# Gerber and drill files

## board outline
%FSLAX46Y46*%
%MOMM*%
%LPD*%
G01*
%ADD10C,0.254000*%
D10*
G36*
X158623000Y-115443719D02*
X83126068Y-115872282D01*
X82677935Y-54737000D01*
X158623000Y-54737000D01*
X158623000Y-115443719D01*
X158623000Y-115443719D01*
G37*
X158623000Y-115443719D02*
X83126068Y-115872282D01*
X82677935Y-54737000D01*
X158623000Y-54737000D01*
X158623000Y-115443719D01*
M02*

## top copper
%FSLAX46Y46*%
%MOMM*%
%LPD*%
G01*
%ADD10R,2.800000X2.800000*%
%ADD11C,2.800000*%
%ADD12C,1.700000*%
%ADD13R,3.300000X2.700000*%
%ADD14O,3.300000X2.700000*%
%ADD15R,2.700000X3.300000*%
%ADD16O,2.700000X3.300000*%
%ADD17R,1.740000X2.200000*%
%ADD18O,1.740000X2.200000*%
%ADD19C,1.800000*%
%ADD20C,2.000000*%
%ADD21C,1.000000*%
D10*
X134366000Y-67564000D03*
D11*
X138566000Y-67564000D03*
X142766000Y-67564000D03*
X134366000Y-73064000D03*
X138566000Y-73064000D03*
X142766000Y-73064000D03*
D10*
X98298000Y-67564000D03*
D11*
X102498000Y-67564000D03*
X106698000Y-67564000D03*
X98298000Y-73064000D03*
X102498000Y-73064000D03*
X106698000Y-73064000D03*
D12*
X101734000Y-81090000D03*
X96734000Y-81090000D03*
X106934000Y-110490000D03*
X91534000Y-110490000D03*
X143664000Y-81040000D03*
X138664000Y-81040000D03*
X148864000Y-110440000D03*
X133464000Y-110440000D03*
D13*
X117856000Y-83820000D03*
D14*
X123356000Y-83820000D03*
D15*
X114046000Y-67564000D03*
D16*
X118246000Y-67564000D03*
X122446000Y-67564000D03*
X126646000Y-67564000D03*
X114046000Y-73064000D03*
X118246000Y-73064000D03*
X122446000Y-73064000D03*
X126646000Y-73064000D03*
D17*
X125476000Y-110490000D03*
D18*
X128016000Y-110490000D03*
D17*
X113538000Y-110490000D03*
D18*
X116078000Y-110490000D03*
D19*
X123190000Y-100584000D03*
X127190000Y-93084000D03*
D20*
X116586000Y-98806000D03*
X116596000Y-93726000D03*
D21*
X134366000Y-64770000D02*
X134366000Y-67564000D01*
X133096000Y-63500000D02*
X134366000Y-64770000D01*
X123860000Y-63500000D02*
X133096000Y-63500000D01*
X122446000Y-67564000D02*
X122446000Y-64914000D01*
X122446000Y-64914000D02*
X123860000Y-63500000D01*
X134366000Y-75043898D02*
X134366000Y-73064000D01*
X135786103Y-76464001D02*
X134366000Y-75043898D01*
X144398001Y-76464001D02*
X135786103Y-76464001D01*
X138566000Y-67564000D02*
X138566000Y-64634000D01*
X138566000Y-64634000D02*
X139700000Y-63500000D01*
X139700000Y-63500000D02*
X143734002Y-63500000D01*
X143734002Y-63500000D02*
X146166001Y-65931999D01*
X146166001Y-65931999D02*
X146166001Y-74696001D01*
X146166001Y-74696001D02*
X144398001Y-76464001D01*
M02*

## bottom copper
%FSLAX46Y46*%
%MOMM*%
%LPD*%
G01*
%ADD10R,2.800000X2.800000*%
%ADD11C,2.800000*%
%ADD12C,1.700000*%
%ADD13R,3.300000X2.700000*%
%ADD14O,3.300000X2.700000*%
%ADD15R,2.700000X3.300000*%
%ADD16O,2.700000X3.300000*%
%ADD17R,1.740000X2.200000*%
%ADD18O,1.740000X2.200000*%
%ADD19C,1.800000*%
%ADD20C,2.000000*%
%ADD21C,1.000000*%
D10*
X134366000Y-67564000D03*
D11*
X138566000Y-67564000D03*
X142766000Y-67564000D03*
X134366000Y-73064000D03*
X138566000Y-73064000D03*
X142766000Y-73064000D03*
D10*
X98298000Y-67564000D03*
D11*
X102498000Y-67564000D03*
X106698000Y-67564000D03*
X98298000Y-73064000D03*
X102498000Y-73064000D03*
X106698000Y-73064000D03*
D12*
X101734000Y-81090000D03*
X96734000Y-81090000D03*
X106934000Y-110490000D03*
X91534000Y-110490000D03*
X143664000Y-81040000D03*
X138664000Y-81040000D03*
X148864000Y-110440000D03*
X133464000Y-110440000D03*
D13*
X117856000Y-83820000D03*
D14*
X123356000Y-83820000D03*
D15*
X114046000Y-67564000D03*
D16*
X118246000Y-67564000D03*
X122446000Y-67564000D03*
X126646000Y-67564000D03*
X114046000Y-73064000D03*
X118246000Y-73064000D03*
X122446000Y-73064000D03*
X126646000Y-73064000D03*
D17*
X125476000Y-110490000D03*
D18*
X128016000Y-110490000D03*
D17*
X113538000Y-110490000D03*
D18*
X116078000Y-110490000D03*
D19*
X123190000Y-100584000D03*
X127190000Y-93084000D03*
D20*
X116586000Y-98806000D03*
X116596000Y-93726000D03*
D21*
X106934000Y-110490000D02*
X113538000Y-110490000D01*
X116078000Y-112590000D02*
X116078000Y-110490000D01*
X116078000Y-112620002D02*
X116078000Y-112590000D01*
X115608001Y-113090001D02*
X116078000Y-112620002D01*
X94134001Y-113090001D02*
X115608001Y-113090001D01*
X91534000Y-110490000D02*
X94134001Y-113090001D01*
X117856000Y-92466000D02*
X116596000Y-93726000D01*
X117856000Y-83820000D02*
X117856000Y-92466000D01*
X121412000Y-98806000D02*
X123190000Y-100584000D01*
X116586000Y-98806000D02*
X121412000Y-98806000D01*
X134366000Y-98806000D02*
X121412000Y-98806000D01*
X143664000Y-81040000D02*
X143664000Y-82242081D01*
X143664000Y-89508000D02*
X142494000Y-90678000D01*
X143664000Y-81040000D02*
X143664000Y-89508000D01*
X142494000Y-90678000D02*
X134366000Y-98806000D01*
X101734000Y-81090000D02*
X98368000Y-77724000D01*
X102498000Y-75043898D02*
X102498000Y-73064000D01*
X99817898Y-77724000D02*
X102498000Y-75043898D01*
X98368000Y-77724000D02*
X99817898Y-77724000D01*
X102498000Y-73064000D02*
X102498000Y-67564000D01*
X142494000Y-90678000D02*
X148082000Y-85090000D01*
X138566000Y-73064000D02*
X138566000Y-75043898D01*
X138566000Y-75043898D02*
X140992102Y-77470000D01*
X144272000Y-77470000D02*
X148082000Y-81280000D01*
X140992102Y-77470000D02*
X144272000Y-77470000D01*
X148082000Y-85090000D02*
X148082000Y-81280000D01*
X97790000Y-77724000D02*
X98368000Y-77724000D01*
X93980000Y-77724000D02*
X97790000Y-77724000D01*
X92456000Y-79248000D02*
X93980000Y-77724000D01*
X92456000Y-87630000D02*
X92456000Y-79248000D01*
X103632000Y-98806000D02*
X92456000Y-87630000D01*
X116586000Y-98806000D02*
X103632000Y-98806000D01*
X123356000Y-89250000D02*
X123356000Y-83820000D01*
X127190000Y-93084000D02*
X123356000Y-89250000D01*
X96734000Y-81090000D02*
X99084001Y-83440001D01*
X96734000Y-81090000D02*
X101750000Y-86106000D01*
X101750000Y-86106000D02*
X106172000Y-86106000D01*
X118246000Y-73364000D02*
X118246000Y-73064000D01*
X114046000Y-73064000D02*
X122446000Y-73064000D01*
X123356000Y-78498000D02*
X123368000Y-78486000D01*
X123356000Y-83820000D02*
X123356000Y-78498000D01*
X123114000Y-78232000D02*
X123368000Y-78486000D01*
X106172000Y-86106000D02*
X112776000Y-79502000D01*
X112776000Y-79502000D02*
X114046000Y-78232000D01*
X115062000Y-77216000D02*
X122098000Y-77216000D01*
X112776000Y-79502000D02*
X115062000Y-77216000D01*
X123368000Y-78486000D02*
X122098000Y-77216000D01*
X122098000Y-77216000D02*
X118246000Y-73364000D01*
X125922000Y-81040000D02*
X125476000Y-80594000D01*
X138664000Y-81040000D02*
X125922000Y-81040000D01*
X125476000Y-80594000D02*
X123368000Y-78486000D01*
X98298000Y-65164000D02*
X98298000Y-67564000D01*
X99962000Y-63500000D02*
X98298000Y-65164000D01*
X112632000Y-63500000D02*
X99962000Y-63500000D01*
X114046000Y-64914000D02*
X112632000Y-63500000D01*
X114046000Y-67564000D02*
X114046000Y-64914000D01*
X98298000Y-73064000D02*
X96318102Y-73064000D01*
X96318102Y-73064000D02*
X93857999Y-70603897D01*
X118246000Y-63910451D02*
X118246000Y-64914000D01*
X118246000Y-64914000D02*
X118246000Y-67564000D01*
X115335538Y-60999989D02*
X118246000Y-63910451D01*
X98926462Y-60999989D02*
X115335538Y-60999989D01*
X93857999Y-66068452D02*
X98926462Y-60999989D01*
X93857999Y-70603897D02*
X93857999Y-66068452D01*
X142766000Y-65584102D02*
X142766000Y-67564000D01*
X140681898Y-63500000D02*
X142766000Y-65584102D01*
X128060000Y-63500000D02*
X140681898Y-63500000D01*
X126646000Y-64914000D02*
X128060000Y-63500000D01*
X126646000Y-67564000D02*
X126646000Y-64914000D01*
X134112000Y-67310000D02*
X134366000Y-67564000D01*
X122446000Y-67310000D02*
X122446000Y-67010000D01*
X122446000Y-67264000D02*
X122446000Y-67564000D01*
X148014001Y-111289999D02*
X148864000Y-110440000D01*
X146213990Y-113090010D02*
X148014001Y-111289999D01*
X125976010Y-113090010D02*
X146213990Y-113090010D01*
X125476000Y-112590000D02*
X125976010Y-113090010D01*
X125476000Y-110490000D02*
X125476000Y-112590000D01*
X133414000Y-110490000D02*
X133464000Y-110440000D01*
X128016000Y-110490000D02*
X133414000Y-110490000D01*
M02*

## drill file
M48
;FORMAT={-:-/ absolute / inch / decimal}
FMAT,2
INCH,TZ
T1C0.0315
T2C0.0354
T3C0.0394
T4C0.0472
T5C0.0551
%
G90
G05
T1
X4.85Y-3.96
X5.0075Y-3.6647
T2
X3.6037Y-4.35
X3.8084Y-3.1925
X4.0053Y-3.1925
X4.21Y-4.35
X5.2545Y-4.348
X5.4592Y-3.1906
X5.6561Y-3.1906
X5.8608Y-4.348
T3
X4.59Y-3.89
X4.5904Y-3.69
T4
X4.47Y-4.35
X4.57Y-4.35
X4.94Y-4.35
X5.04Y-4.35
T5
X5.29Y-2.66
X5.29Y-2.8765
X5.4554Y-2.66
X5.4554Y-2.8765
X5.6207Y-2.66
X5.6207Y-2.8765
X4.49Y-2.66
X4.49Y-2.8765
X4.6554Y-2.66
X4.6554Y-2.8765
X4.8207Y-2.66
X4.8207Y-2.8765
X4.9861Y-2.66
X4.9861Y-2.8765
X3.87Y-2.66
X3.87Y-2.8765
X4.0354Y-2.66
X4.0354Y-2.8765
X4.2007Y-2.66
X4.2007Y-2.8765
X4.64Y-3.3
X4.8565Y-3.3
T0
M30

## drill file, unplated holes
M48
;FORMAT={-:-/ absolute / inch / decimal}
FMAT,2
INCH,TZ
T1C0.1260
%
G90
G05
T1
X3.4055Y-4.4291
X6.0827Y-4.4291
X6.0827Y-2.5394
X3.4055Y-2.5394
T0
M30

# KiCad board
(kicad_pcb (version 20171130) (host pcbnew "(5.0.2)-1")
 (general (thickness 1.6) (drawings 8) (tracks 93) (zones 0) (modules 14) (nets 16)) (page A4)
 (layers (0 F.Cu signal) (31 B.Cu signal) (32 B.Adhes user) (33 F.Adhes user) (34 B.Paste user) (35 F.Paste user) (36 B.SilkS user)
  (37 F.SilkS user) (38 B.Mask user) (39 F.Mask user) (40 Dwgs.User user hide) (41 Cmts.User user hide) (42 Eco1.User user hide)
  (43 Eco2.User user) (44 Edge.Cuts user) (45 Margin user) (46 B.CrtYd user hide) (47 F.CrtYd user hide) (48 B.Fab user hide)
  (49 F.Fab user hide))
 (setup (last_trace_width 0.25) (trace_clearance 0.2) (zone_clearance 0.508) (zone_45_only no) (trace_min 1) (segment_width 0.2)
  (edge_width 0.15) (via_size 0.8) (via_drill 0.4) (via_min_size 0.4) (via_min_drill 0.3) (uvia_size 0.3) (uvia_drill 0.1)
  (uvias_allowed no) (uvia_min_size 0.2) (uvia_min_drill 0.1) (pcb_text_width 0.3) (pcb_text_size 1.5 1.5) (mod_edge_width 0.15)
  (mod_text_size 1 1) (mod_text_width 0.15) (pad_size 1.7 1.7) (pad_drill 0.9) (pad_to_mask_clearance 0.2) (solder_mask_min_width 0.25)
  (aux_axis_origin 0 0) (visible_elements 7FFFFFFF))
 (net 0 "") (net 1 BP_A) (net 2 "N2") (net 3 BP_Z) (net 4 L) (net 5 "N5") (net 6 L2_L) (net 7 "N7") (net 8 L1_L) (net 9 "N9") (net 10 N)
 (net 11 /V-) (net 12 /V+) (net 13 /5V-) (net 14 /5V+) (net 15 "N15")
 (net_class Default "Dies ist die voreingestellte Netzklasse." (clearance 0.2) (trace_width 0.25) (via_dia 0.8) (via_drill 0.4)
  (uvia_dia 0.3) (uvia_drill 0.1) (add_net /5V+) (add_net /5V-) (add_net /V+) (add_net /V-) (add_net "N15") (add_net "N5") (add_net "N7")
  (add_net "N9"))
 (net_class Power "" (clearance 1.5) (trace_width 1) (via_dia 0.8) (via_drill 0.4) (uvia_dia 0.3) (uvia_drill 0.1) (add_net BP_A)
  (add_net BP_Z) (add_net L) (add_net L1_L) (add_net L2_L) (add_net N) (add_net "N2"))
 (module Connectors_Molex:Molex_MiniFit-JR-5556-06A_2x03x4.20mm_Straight (layer F.Cu) (at 134.366 67.564)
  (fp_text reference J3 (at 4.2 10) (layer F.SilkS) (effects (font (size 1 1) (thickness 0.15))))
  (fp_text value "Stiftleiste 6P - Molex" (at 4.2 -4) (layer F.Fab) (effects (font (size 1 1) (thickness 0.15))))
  (pad 1 thru_hole rect (at 0 0) (size 2.8 2.8) (drill 1.4) (layers *.Cu *.Mask) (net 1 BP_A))
  (pad 2 thru_hole circle (at 4.2 0) (size 2.8 2.8) (drill 1.4) (layers *.Cu *.Mask) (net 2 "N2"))
  (pad 3 thru_hole circle (at 8.4 0) (size 2.8 2.8) (drill 1.4) (layers *.Cu *.Mask) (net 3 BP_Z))
  (pad 4 thru_hole circle (at 0 5.5) (size 2.8 2.8) (drill 1.4) (layers *.Cu *.Mask) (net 2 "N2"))
  (pad 5 thru_hole circle (at 4.2 5.5) (size 2.8 2.8) (drill 1.4) (layers *.Cu *.Mask) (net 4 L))
  (pad 6 thru_hole circle (at 8.4 5.5) (size 2.8 2.8) (drill 1.4) (layers *.Cu *.Mask) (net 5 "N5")))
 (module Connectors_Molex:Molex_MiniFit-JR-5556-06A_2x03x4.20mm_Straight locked (layer F.Cu) (at 98.298 67.564)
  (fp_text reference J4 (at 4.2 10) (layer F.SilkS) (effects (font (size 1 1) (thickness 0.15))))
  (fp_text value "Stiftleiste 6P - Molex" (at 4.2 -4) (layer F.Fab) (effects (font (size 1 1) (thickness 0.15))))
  (pad 1 thru_hole rect (at 0 0) (size 2.8 2.8) (drill 1.4) (layers *.Cu *.Mask) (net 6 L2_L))
  (pad 2 thru_hole circle (at 4.2 0) (size 2.8 2.8) (drill 1.4) (layers *.Cu *.Mask) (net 4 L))
  (pad 3 thru_hole circle (at 8.4 0) (size 2.8 2.8) (drill 1.4) (layers *.Cu *.Mask) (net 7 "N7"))
  (pad 4 thru_hole circle (at 0 5.5) (size 2.8 2.8) (drill 1.4) (layers *.Cu *.Mask) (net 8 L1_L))
  (pad 5 thru_hole circle (at 4.2 5.5) (size 2.8 2.8) (drill 1.4) (layers *.Cu *.Mask) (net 4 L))
  (pad 6 thru_hole circle (at 8.4 5.5) (size 2.8 2.8) (drill 1.4) (layers *.Cu *.Mask) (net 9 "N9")))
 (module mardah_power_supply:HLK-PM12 (layer F.Cu) (at 89.134 78.79 270)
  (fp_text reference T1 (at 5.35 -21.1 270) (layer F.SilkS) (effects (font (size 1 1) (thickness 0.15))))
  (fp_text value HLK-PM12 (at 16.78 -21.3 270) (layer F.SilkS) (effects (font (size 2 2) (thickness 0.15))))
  (pad 1 thru_hole circle (at 2.3 -12.6 270) (size 1.7 1.7) (drill 0.9) (layers *.Cu *.Mask F.SilkS) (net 4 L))
  (pad 2 thru_hole circle (at 2.3 -7.6 270) (size 1.7 1.7) (drill 0.9) (layers *.Cu *.Mask F.SilkS) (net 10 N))
  (pad 3 thru_hole circle (at 31.7 -17.8 270) (size 1.7 1.7) (drill 0.9) (layers *.Cu *.Mask F.SilkS) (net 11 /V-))
  (pad 4 thru_hole circle (at 31.7 -2.4 270) (size 1.7 1.7) (drill 0.9) (layers *.Cu *.Mask F.SilkS) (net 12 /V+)))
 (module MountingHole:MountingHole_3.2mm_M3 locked (layer F.Cu) (at 154.5 64.5)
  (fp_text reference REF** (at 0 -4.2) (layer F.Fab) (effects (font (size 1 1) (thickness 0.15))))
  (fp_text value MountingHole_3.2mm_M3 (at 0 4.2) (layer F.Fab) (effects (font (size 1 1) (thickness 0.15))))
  (pad 1 np_thru_hole circle (at 0 0) (size 3.2 3.2) (drill 3.2) (layers *.Cu *.Mask)))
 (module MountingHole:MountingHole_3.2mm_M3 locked (layer F.Cu) (at 154.5 112.5)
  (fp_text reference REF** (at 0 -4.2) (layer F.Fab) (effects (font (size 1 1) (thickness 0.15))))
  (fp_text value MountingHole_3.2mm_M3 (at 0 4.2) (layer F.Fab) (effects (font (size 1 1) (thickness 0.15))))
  (pad 1 np_thru_hole circle (at 0 0) (size 3.2 3.2) (drill 3.2) (layers *.Cu *.Mask)))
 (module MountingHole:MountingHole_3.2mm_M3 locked (layer F.Cu) (at 86.5 112.5)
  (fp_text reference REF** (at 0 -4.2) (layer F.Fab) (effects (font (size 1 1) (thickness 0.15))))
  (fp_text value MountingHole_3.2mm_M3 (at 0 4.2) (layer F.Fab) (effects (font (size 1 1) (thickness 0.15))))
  (pad 1 np_thru_hole circle (at 0 0) (size 3.2 3.2) (drill 3.2) (layers *.Cu *.Mask)))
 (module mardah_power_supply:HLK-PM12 (layer F.Cu) (at 131.064 78.74 270)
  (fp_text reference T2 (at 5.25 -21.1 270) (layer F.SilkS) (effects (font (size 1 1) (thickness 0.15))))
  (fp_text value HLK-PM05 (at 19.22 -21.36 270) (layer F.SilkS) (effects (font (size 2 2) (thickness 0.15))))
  (pad 1 thru_hole circle (at 2.3 -12.6 270) (size 1.7 1.7) (drill 0.9) (layers *.Cu *.Mask F.SilkS) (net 4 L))
  (pad 2 thru_hole circle (at 2.3 -7.6 270) (size 1.7 1.7) (drill 0.9) (layers *.Cu *.Mask F.SilkS) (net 10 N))
  (pad 3 thru_hole circle (at 31.7 -17.8 270) (size 1.7 1.7) (drill 0.9) (layers *.Cu *.Mask F.SilkS) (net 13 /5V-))
  (pad 4 thru_hole circle (at 31.7 -2.4 270) (size 1.7 1.7) (drill 0.9) (layers *.Cu *.Mask F.SilkS) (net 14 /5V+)))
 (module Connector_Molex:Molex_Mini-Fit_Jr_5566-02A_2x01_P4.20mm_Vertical (layer F.Cu) (at 117.856 83.82 90)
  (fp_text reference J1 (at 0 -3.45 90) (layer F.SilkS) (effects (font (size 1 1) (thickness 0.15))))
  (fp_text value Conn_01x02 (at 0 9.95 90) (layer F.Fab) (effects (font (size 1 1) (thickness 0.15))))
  (pad 1 thru_hole rect (at 0 0 90) (size 2.7 3.3) (drill 1.4) (layers *.Cu *.Mask) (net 4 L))
  (pad 2 thru_hole oval (at 0 5.5 90) (size 2.7 3.3) (drill 1.4) (layers *.Cu *.Mask) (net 10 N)))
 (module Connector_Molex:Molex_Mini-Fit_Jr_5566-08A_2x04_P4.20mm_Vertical (layer F.Cu) (at 114.046 67.564)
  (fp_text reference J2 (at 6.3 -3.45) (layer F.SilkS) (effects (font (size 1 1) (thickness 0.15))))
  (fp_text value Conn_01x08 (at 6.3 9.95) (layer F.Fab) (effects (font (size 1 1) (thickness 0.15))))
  (pad 1 thru_hole rect (at 0 0) (size 2.7 3.3) (drill 1.4) (layers *.Cu *.Mask) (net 6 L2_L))
  (pad 2 thru_hole oval (at 4.2 0) (size 2.7 3.3) (drill 1.4) (layers *.Cu *.Mask) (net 8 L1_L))
  (pad 3 thru_hole oval (at 8.4 0) (size 2.7 3.3) (drill 1.4) (layers *.Cu *.Mask) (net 1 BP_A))
  (pad 4 thru_hole oval (at 12.6 0) (size 2.7 3.3) (drill 1.4) (layers *.Cu *.Mask) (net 3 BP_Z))
  (pad 5 thru_hole oval (at 0 5.5) (size 2.7 3.3) (drill 1.4) (layers *.Cu *.Mask) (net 10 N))
  (pad 6 thru_hole oval (at 4.2 5.5) (size 2.7 3.3) (drill 1.4) (layers *.Cu *.Mask) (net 10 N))
  (pad 7 thru_hole oval (at 8.4 5.5) (size 2.7 3.3) (drill 1.4) (layers *.Cu *.Mask) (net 10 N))
  (pad 8 thru_hole oval (at 12.6 5.5) (size 2.7 3.3) (drill 1.4) (layers *.Cu *.Mask) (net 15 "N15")))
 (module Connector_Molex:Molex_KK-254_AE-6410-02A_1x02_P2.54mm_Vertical (layer F.Cu) (at 125.476 110.49)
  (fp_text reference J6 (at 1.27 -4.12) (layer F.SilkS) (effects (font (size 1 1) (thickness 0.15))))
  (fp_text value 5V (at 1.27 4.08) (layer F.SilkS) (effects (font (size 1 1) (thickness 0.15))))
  (pad 1 thru_hole rect (at 0 0) (size 1.74 2.2) (drill 1.2) (layers *.Cu *.Mask) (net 13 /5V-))
  (pad 2 thru_hole oval (at 2.54 0) (size 1.74 2.2) (drill 1.2) (layers *.Cu *.Mask) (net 14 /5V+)))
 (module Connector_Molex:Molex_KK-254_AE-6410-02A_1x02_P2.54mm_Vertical (layer F.Cu) (at 113.538 110.49)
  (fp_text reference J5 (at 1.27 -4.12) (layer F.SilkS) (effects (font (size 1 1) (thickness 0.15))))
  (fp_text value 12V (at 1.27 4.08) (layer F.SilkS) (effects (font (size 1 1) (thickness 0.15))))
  (pad 1 thru_hole rect (at 0 0) (size 1.74 2.2) (drill 1.2) (layers *.Cu *.Mask) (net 11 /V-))
  (pad 2 thru_hole oval (at 2.54 0) (size 1.74 2.2) (drill 1.2) (layers *.Cu *.Mask) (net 12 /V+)))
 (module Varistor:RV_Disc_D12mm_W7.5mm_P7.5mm (layer F.Cu) (at 123.19 100.584 90)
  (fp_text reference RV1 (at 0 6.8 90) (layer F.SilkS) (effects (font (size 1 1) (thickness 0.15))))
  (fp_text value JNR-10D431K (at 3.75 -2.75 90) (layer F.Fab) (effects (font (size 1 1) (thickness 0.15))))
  (pad 1 thru_hole circle (at 0 0 90) (size 1.8 1.8) (drill 0.8) (layers *.Cu *.Mask) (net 4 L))
  (pad 2 thru_hole circle (at 7.5 4 90) (size 1.8 1.8) (drill 0.8) (layers *.Cu *.Mask) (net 10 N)))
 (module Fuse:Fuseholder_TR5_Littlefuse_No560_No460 (layer F.Cu) (at 116.586 98.806 90)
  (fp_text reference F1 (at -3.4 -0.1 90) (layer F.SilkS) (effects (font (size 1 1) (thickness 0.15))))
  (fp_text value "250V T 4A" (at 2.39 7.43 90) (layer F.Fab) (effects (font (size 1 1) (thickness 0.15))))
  (pad 1 thru_hole circle (at 0 0 90) (size 2 2) (drill 1) (layers *.Cu *.Mask) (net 4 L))
  (pad 2 thru_hole circle (at 5.08 0.01 90) (size 2 2) (drill 1) (layers *.Cu *.Mask) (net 4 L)))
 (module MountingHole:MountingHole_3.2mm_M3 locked (layer F.Cu) (at 86.5 64.5)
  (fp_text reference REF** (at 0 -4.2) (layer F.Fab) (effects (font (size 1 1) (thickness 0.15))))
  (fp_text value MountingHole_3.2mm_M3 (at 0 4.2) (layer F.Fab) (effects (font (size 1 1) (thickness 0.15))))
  (pad 1 np_thru_hole circle (at 0 0) (size 3.2 3.2) (drill 3.2) (layers *.Cu *.Mask)))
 (segment (start 106.934 110.49) (end 113.538 110.49) (width 1) (layer B.Cu) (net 11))
 (segment (start 116.078 112.59) (end 116.078 110.49) (width 1) (layer B.Cu) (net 12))
 (segment (start 116.078 112.620002) (end 116.078 112.59) (width 1) (layer B.Cu) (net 12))
 (segment (start 115.608001 113.090001) (end 116.078 112.620002) (width 1) (layer B.Cu) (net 12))
 (segment (start 94.134001 113.090001) (end 115.608001 113.090001) (width 1) (layer B.Cu) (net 12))
 (segment (start 91.534 110.49) (end 94.134001 113.090001) (width 1) (layer B.Cu) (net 12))
 (segment (start 117.856 92.466) (end 116.596 93.726) (width 1) (layer B.Cu) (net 4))
 (segment (start 117.856 83.82) (end 117.856 92.466) (width 1) (layer B.Cu) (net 4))
 (segment (start 121.412 98.806) (end 123.19 100.584) (width 1) (layer B.Cu) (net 4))
 (segment (start 116.586 98.806) (end 121.412 98.806) (width 1) (layer B.Cu) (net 4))
 (segment (start 134.366 98.806) (end 121.412 98.806) (width 1) (layer B.Cu) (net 4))
 (segment (start 143.664 81.04) (end 143.664 82.242081) (width 1) (layer B.Cu) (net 4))
 (segment (start 143.664 89.508) (end 142.494 90.678) (width 1) (layer B.Cu) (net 4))
 (segment (start 143.664 81.04) (end 143.664 89.508) (width 1) (layer B.Cu) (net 4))
 (segment (start 142.494 90.678) (end 134.366 98.806) (width 1) (layer B.Cu) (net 4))
 (segment (start 101.734 81.09) (end 98.368 77.724) (width 1) (layer B.Cu) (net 4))
 (segment (start 102.498 75.043898) (end 102.498 73.064) (width 1) (layer B.Cu) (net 4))
 (segment (start 99.817898 77.724) (end 102.498 75.043898) (width 1) (layer B.Cu) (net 4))
 (segment (start 98.368 77.724) (end 99.817898 77.724) (width 1) (layer B.Cu) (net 4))
 (segment (start 102.498 73.064) (end 102.498 67.564) (width 1) (layer B.Cu) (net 4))
 (segment (start 142.494 90.678) (end 148.082 85.09) (width 1) (layer B.Cu) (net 4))
 (segment (start 138.566 73.064) (end 138.566 75.043898) (width 1) (layer B.Cu) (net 4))
 (segment (start 138.566 75.043898) (end 140.992102 77.47) (width 1) (layer B.Cu) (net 4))
 (segment (start 144.272 77.47) (end 148.082 81.28) (width 1) (layer B.Cu) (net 4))
 (segment (start 140.992102 77.47) (end 144.272 77.47) (width 1) (layer B.Cu) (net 4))
 (segment (start 148.082 85.09) (end 148.082 81.28) (width 1) (layer B.Cu) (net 4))
 (segment (start 97.79 77.724) (end 98.368 77.724) (width 1) (layer B.Cu) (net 4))
 (segment (start 93.98 77.724) (end 97.79 77.724) (width 1) (layer B.Cu) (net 4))
 (segment (start 92.456 79.248) (end 93.98 77.724) (width 1) (layer B.Cu) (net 4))
 (segment (start 92.456 87.63) (end 92.456 79.248) (width 1) (layer B.Cu) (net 4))
 (segment (start 103.632 98.806) (end 92.456 87.63) (width 1) (layer B.Cu) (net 4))
 (segment (start 116.586 98.806) (end 103.632 98.806) (width 1) (layer B.Cu) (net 4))
 (segment (start 123.356 89.25) (end 123.356 83.82) (width 1) (layer B.Cu) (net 10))
 (segment (start 127.19 93.084) (end 123.356 89.25) (width 1) (layer B.Cu) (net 10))
 (segment (start 96.734 81.09) (end 99.084001 83.440001) (width 1) (layer B.Cu) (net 10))
 (segment (start 96.734 81.09) (end 101.75 86.106) (width 1) (layer B.Cu) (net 10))
 (segment (start 101.75 86.106) (end 106.172 86.106) (width 1) (layer B.Cu) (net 10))
 (segment (start 118.246 73.364) (end 118.246 73.064) (width 1) (layer B.Cu) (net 10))
 (segment (start 114.046 73.064) (end 122.446 73.064) (width 1) (layer B.Cu) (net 10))
 (segment (start 123.356 78.498) (end 123.368 78.486) (width 1) (layer B.Cu) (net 10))
 (segment (start 123.356 83.82) (end 123.356 78.498) (width 1) (layer B.Cu) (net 10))
 (segment (start 123.114 78.232) (end 123.368 78.486) (width 1) (layer B.Cu) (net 10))
 (segment (start 106.172 86.106) (end 112.776 79.502) (width 1) (layer B.Cu) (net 10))
 (segment (start 112.776 79.502) (end 114.046 78.232) (width 1) (layer B.Cu) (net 10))
 (segment (start 115.062 77.216) (end 122.098 77.216) (width 1) (layer B.Cu) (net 10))
 (segment (start 112.776 79.502) (end 115.062 77.216) (width 1) (layer B.Cu) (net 10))
 (segment (start 123.368 78.486) (end 122.098 77.216) (width 1) (layer B.Cu) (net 10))
 (segment (start 122.098 77.216) (end 118.246 73.364) (width 1) (layer B.Cu) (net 10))
 (segment (start 125.922 81.04) (end 125.476 80.594) (width 1) (layer B.Cu) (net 10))
 (segment (start 138.664 81.04) (end 125.922 81.04) (width 1) (layer B.Cu) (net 10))
 (segment (start 125.476 80.594) (end 123.368 78.486) (width 1) (layer B.Cu) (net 10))
 (segment (start 98.298 65.164) (end 98.298 67.564) (width 1) (layer B.Cu) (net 6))
 (segment (start 99.962 63.5) (end 98.298 65.164) (width 1) (layer B.Cu) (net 6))
 (segment (start 112.632 63.5) (end 99.962 63.5) (width 1) (layer B.Cu) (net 6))
 (segment (start 114.046 64.914) (end 112.632 63.5) (width 1) (layer B.Cu) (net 6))
 (segment (start 114.046 67.564) (end 114.046 64.914) (width 1) (layer B.Cu) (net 6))
 (segment (start 98.298 73.064) (end 96.318102 73.064) (width 1) (layer B.Cu) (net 8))
 (segment (start 96.318102 73.064) (end 93.857999 70.603897) (width 1) (layer B.Cu) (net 8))
 (segment (start 118.246 63.910451) (end 118.246 64.914) (width 1) (layer B.Cu) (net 8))
 (segment (start 118.246 64.914) (end 118.246 67.564) (width 1) (layer B.Cu) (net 8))
 (segment (start 115.335538 60.999989) (end 118.246 63.910451) (width 1) (layer B.Cu) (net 8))
 (segment (start 98.926462 60.999989) (end 115.335538 60.999989) (width 1) (layer B.Cu) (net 8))
 (segment (start 93.857999 66.068452) (end 98.926462 60.999989) (width 1) (layer B.Cu) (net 8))
 (segment (start 93.857999 70.603897) (end 93.857999 66.068452) (width 1) (layer B.Cu) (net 8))
 (segment (start 142.766 65.584102) (end 142.766 67.564) (width 1) (layer B.Cu) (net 3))
 (segment (start 140.681898 63.5) (end 142.766 65.584102) (width 1) (layer B.Cu) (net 3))
 (segment (start 128.06 63.5) (end 140.681898 63.5) (width 1) (layer B.Cu) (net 3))
 (segment (start 126.646 64.914) (end 128.06 63.5) (width 1) (layer B.Cu) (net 3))
 (segment (start 126.646 67.564) (end 126.646 64.914) (width 1) (layer B.Cu) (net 3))
 (segment (start 134.112 67.31) (end 134.366 67.564) (width 1) (layer B.Cu) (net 1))
 (segment (start 122.446 67.31) (end 122.446 67.01) (width 1) (layer B.Cu) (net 1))
 (segment (start 122.446 67.264) (end 122.446 67.564) (width 1) (layer B.Cu) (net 1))
 (segment (start 134.366 64.77) (end 134.366 67.564) (width 1) (layer F.Cu) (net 1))
 (segment (start 133.096 63.5) (end 134.366 64.77) (width 1) (layer F.Cu) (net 1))
 (segment (start 123.86 63.5) (end 133.096 63.5) (width 1) (layer F.Cu) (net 1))
 (segment (start 122.446 67.564) (end 122.446 64.914) (width 1) (layer F.Cu) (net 1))
 (segment (start 122.446 64.914) (end 123.86 63.5) (width 1) (layer F.Cu) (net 1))
 (segment (start 148.014001 111.289999) (end 148.864 110.44) (width 1) (layer B.Cu) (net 13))
 (segment (start 146.21399 113.09001) (end 148.014001 111.289999) (width 1) (layer B.Cu) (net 13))
 (segment (start 125.97601 113.09001) (end 146.21399 113.09001) (width 1) (layer B.Cu) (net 13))
 (segment (start 125.476 112.59) (end 125.97601 113.09001) (width 1) (layer B.Cu) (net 13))
 (segment (start 125.476 110.49) (end 125.476 112.59) (width 1) (layer B.Cu) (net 13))
 (segment (start 133.414 110.49) (end 133.464 110.44) (width 1) (layer B.Cu) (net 14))
 (segment (start 128.016 110.49) (end 133.414 110.49) (width 1) (layer B.Cu) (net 14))
 (segment (start 134.366 75.043898) (end 134.366 73.064) (width 1) (layer F.Cu) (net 2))
 (segment (start 135.786103 76.464001) (end 134.366 75.043898) (width 1) (layer F.Cu) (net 2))
 (segment (start 144.398001 76.464001) (end 135.786103 76.464001) (width 1) (layer F.Cu) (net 2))
 (segment (start 138.566 67.564) (end 138.566 64.634) (width 1) (layer F.Cu) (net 2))
 (segment (start 138.566 64.634) (end 139.7 63.5) (width 1) (layer F.Cu) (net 2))
 (segment (start 139.7 63.5) (end 143.734002 63.5) (width 1) (layer F.Cu) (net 2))
 (segment (start 143.734002 63.5) (end 146.166001 65.931999) (width 1) (layer F.Cu) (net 2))
 (segment (start 146.166001 65.931999) (end 146.166001 74.696001) (width 1) (layer F.Cu) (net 2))
 (segment (start 146.166001 74.696001) (end 144.398001 76.464001) (width 1) (layer F.Cu) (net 2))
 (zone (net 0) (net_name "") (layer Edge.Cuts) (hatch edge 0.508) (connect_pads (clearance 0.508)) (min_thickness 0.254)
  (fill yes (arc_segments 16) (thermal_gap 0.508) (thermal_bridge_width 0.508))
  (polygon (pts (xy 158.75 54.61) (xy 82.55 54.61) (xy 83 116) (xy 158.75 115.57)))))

